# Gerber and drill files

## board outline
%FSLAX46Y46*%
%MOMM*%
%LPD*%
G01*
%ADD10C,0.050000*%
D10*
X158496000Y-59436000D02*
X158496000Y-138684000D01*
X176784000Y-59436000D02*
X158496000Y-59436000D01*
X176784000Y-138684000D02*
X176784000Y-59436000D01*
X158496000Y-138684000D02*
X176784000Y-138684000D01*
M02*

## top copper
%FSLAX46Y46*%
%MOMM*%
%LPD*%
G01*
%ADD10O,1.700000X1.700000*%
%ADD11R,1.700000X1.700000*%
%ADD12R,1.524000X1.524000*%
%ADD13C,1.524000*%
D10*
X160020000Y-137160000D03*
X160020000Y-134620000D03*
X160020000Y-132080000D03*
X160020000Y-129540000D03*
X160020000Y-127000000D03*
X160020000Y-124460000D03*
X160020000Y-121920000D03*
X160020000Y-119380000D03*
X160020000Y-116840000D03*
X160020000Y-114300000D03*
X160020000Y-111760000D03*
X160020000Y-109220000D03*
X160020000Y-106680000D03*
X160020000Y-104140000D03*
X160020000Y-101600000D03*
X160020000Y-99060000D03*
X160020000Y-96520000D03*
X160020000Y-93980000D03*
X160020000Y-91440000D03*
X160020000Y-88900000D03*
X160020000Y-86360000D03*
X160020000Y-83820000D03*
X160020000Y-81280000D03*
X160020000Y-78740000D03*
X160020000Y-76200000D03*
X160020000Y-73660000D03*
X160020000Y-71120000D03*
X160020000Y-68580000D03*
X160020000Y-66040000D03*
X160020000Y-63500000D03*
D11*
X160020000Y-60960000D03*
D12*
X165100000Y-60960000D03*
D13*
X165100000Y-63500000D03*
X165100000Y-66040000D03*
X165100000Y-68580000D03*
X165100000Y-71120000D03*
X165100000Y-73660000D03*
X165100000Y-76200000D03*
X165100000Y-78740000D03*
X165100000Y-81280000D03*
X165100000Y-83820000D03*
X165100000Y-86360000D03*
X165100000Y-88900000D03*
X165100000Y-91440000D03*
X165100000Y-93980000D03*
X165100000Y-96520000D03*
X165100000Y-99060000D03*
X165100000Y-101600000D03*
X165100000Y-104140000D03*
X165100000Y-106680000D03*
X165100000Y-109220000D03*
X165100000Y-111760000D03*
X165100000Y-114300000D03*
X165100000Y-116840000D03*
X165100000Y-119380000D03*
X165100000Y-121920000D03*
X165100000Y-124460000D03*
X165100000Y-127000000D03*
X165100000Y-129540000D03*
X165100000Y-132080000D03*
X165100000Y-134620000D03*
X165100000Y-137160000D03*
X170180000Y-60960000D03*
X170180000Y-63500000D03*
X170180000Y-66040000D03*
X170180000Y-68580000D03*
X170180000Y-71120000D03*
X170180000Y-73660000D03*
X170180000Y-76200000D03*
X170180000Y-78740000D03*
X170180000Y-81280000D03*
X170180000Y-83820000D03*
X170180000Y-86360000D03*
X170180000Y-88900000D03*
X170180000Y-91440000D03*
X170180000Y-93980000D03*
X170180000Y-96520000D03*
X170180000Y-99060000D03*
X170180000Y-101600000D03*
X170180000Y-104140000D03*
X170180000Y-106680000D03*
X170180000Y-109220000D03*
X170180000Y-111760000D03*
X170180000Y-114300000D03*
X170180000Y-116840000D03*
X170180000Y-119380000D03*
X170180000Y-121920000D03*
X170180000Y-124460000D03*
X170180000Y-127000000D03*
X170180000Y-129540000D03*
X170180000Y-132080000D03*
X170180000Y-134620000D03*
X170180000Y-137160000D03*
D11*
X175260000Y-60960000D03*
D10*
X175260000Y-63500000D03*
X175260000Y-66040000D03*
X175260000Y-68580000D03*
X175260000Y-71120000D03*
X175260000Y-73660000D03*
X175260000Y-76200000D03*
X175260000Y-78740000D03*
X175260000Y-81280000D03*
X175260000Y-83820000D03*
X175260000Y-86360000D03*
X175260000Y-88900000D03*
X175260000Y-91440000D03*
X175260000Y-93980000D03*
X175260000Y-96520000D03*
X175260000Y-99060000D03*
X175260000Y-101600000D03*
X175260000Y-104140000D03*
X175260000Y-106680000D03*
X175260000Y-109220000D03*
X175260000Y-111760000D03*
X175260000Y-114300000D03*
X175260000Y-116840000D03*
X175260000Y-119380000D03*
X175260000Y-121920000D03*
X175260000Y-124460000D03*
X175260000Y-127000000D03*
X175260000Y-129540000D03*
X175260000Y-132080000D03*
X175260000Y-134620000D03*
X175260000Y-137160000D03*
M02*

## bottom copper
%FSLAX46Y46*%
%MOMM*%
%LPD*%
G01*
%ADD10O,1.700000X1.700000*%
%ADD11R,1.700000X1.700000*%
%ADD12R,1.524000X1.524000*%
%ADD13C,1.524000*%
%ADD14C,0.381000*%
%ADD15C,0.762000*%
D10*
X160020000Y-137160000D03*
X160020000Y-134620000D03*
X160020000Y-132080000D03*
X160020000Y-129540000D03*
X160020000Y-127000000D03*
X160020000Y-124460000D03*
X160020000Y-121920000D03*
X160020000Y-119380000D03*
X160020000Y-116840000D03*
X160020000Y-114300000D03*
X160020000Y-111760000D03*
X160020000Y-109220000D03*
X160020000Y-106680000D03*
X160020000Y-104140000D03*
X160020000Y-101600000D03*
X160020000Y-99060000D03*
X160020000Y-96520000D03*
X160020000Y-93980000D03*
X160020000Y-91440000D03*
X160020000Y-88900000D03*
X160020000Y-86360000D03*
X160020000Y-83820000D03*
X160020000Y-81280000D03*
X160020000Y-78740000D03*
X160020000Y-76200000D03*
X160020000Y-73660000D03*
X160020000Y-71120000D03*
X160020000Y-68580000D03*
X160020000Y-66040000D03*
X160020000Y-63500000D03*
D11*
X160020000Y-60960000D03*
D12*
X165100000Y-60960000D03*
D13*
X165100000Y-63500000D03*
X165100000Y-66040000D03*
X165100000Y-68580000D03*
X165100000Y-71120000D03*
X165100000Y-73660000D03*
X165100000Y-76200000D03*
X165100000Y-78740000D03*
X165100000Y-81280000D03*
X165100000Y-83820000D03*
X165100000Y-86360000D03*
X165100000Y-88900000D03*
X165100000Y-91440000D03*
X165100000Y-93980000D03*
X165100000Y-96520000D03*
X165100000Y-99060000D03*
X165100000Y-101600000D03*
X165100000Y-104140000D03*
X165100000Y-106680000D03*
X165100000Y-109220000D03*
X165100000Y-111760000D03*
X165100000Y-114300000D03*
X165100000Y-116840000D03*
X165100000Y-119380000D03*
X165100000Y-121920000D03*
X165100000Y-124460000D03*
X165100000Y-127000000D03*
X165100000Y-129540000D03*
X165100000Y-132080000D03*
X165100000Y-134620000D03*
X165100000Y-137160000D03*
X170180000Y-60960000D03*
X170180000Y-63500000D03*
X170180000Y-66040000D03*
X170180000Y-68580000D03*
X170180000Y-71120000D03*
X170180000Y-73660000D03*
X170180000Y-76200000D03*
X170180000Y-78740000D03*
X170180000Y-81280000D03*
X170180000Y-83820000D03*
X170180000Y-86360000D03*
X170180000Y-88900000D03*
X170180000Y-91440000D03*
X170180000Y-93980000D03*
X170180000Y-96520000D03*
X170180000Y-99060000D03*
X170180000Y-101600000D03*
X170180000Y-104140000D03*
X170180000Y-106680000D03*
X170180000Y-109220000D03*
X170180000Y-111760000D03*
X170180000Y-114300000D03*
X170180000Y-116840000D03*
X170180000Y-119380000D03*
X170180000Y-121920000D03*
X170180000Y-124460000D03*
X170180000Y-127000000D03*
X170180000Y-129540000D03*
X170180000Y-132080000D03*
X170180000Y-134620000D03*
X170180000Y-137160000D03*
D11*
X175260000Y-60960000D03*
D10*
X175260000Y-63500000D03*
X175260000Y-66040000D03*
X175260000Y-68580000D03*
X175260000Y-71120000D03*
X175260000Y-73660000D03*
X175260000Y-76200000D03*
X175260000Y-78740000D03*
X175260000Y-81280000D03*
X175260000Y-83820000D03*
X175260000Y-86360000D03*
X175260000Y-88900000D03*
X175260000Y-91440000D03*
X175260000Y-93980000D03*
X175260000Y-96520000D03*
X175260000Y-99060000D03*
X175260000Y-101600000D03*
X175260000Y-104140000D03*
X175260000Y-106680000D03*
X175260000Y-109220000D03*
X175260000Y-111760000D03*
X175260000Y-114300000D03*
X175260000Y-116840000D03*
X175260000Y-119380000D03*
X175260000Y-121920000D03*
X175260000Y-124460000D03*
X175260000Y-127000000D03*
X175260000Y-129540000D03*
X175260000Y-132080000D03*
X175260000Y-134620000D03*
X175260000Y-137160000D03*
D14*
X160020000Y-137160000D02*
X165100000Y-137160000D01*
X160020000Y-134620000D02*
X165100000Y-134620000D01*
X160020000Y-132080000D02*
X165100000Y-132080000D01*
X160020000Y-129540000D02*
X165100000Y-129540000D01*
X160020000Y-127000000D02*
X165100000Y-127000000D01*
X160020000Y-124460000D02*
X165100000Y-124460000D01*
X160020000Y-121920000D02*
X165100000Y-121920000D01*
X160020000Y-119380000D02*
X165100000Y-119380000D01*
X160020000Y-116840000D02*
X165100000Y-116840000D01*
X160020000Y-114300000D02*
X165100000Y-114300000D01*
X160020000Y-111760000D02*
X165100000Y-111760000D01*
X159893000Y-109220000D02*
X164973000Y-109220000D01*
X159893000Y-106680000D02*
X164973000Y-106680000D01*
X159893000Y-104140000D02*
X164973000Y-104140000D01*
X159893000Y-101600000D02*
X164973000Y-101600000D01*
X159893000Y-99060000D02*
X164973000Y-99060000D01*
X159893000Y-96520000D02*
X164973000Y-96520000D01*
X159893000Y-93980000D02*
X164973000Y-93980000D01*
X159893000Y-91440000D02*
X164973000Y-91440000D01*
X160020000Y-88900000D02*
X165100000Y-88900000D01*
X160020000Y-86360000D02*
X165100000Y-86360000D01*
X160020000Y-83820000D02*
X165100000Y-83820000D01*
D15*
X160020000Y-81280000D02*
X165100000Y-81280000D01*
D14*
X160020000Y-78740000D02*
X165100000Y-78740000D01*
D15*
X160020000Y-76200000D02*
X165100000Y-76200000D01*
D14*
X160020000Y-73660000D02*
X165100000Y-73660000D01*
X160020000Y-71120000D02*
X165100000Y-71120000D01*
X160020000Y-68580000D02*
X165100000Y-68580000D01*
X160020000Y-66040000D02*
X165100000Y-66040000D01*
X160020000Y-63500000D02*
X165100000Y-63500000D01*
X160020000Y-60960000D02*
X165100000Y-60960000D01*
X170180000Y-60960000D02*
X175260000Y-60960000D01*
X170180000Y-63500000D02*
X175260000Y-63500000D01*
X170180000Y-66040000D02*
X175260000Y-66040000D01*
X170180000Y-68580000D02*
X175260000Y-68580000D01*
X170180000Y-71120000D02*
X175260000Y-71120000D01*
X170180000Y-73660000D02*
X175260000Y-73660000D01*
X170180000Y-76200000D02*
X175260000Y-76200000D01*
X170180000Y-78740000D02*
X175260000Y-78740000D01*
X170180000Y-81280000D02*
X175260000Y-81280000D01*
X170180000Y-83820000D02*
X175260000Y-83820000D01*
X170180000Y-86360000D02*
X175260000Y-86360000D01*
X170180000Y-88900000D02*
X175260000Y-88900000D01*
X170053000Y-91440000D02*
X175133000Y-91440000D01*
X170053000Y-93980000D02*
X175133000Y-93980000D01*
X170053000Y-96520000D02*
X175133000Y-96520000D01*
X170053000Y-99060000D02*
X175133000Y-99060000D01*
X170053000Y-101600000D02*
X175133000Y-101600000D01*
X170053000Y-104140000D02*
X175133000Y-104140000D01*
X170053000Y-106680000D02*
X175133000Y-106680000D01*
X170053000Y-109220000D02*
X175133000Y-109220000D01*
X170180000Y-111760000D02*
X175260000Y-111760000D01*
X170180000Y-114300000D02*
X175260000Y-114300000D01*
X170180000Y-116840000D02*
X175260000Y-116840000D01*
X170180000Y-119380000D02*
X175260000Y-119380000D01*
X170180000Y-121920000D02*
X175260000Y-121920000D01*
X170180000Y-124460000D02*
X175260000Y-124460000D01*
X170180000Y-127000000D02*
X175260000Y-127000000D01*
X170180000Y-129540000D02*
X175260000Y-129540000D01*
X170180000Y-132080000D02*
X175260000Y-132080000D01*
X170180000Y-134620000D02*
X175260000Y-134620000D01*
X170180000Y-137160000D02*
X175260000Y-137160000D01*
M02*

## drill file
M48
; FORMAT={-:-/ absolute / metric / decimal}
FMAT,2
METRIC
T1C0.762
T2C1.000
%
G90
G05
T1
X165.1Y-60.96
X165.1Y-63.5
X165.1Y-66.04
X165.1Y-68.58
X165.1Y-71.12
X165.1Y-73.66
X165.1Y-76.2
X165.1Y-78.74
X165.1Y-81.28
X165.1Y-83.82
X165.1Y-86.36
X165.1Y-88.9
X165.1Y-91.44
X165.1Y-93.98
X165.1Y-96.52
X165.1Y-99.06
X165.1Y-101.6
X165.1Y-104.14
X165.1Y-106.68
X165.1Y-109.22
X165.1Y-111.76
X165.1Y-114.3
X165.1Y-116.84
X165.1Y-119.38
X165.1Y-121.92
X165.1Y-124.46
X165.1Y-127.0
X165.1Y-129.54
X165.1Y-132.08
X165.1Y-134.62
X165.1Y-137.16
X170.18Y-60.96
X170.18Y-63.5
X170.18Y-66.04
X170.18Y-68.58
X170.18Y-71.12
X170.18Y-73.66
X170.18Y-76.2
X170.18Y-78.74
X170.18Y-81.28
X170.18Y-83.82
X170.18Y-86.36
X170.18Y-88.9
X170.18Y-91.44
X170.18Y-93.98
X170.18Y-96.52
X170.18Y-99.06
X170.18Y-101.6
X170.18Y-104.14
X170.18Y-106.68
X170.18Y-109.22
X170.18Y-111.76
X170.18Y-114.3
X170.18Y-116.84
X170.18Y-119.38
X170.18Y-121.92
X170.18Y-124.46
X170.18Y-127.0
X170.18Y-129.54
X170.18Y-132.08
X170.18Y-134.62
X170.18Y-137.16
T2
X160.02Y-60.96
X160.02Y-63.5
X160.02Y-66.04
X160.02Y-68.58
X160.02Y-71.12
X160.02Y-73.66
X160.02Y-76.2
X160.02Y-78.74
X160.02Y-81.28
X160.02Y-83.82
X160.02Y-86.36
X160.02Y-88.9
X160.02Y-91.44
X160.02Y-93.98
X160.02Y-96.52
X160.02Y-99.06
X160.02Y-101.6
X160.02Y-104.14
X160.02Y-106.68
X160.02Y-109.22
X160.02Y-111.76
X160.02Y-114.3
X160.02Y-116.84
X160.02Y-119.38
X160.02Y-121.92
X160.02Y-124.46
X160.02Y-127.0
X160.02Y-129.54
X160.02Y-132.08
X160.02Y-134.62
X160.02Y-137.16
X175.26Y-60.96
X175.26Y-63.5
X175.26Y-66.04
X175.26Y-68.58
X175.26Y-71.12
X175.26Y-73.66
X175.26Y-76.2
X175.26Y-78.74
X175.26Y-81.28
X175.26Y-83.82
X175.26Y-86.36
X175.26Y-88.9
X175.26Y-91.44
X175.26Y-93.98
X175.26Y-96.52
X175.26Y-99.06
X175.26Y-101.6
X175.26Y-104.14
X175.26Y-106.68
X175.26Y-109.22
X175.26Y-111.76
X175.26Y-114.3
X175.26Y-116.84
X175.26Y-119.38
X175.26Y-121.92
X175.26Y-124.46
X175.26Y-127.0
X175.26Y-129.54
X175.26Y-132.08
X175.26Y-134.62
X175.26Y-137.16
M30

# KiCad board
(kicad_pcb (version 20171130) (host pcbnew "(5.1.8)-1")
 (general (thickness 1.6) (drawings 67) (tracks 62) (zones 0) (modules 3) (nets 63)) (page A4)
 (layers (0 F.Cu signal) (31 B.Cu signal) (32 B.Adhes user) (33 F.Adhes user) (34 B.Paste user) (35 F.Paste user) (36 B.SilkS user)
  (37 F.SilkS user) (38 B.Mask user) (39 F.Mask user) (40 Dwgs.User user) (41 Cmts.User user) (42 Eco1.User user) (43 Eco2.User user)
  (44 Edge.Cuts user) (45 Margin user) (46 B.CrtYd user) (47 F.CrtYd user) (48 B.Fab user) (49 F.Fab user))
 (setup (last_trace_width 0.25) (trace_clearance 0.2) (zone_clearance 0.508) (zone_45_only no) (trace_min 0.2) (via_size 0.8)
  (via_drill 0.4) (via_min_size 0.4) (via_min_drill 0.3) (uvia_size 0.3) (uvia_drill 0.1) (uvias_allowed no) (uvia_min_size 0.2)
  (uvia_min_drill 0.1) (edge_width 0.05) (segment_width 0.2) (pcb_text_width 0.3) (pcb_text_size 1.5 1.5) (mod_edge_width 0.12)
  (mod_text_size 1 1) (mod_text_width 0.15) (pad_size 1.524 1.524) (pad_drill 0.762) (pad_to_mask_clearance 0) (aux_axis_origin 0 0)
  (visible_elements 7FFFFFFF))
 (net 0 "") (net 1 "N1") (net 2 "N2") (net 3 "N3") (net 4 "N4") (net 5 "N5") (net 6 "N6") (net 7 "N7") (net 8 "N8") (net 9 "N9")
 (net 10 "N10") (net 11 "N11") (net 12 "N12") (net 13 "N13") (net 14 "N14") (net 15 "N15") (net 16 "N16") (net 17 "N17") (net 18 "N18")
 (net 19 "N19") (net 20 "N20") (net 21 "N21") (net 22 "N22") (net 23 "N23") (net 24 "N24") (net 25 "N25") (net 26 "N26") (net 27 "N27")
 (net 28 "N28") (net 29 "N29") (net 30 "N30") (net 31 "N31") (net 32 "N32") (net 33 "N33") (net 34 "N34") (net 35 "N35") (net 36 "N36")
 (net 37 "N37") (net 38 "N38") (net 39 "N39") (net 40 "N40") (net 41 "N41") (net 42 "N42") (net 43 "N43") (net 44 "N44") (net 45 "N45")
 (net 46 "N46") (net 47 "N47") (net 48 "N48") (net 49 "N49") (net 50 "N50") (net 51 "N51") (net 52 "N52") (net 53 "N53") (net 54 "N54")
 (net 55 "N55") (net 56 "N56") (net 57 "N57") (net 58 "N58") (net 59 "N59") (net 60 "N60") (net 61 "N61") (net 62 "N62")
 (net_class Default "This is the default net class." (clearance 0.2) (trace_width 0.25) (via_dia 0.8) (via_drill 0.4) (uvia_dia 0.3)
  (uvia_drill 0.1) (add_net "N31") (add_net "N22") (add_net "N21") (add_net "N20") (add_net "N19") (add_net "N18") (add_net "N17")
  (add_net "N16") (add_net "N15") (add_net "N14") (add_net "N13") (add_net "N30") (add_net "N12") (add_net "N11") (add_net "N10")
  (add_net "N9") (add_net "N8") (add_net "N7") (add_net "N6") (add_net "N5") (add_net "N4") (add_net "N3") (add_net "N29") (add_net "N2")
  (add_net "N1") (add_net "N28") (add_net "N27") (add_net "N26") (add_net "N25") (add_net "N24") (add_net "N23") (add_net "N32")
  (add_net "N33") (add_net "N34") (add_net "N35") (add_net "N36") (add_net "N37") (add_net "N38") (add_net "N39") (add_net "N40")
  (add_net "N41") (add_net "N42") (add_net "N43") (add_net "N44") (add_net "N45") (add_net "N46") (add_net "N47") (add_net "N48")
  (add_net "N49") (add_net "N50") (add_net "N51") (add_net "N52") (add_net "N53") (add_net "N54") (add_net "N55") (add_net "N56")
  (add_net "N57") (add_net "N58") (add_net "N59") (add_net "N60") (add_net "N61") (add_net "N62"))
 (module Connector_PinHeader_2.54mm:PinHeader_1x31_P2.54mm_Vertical (layer B.Cu) (at 160.02 60.96 180)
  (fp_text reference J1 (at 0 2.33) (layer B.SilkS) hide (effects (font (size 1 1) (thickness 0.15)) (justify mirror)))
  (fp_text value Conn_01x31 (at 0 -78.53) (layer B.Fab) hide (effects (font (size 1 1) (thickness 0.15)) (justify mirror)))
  (pad 31 thru_hole oval (at 0 -76.2 180) (size 1.7 1.7) (drill 1) (layers *.Cu *.Mask) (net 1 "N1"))
  (pad 30 thru_hole oval (at 0 -73.66 180) (size 1.7 1.7) (drill 1) (layers *.Cu *.Mask) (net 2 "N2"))
  (pad 29 thru_hole oval (at 0 -71.12 180) (size 1.7 1.7) (drill 1) (layers *.Cu *.Mask) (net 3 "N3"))
  (pad 28 thru_hole oval (at 0 -68.58 180) (size 1.7 1.7) (drill 1) (layers *.Cu *.Mask) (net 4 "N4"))
  (pad 27 thru_hole oval (at 0 -66.04 180) (size 1.7 1.7) (drill 1) (layers *.Cu *.Mask) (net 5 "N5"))
  (pad 26 thru_hole oval (at 0 -63.5 180) (size 1.7 1.7) (drill 1) (layers *.Cu *.Mask) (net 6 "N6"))
  (pad 25 thru_hole oval (at 0 -60.96 180) (size 1.7 1.7) (drill 1) (layers *.Cu *.Mask) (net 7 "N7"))
  (pad 24 thru_hole oval (at 0 -58.42 180) (size 1.7 1.7) (drill 1) (layers *.Cu *.Mask) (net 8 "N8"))
  (pad 23 thru_hole oval (at 0 -55.88 180) (size 1.7 1.7) (drill 1) (layers *.Cu *.Mask) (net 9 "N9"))
  (pad 22 thru_hole oval (at 0 -53.34 180) (size 1.7 1.7) (drill 1) (layers *.Cu *.Mask) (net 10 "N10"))
  (pad 21 thru_hole oval (at 0 -50.8 180) (size 1.7 1.7) (drill 1) (layers *.Cu *.Mask) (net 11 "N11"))
  (pad 20 thru_hole oval (at 0 -48.26 180) (size 1.7 1.7) (drill 1) (layers *.Cu *.Mask) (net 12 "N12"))
  (pad 19 thru_hole oval (at 0 -45.72 180) (size 1.7 1.7) (drill 1) (layers *.Cu *.Mask) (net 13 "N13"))
  (pad 18 thru_hole oval (at 0 -43.18 180) (size 1.7 1.7) (drill 1) (layers *.Cu *.Mask) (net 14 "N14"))
  (pad 17 thru_hole oval (at 0 -40.64 180) (size 1.7 1.7) (drill 1) (layers *.Cu *.Mask) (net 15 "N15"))
  (pad 16 thru_hole oval (at 0 -38.1 180) (size 1.7 1.7) (drill 1) (layers *.Cu *.Mask) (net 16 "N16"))
  (pad 15 thru_hole oval (at 0 -35.56 180) (size 1.7 1.7) (drill 1) (layers *.Cu *.Mask) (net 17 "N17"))
  (pad 14 thru_hole oval (at 0 -33.02 180) (size 1.7 1.7) (drill 1) (layers *.Cu *.Mask) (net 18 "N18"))
  (pad 13 thru_hole oval (at 0 -30.48 180) (size 1.7 1.7) (drill 1) (layers *.Cu *.Mask) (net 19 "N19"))
  (pad 12 thru_hole oval (at 0 -27.94 180) (size 1.7 1.7) (drill 1) (layers *.Cu *.Mask) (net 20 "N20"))
  (pad 11 thru_hole oval (at 0 -25.4 180) (size 1.7 1.7) (drill 1) (layers *.Cu *.Mask) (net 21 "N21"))
  (pad 10 thru_hole oval (at 0 -22.86 180) (size 1.7 1.7) (drill 1) (layers *.Cu *.Mask) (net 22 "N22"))
  (pad 9 thru_hole oval (at 0 -20.32 180) (size 1.7 1.7) (drill 1) (layers *.Cu *.Mask) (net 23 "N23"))
  (pad 8 thru_hole oval (at 0 -17.78 180) (size 1.7 1.7) (drill 1) (layers *.Cu *.Mask) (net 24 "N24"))
  (pad 7 thru_hole oval (at 0 -15.24 180) (size 1.7 1.7) (drill 1) (layers *.Cu *.Mask) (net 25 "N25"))
  (pad 6 thru_hole oval (at 0 -12.7 180) (size 1.7 1.7) (drill 1) (layers *.Cu *.Mask) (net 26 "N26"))
  (pad 5 thru_hole oval (at 0 -10.16 180) (size 1.7 1.7) (drill 1) (layers *.Cu *.Mask) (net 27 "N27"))
  (pad 4 thru_hole oval (at 0 -7.62 180) (size 1.7 1.7) (drill 1) (layers *.Cu *.Mask) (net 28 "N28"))
  (pad 3 thru_hole oval (at 0 -5.08 180) (size 1.7 1.7) (drill 1) (layers *.Cu *.Mask) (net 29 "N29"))
  (pad 2 thru_hole oval (at 0 -2.54 180) (size 1.7 1.7) (drill 1) (layers *.Cu *.Mask) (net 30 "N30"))
  (pad 1 thru_hole rect (at 0 0 180) (size 1.7 1.7) (drill 1) (layers *.Cu *.Mask) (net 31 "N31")))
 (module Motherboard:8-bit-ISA (layer F.Cu) (at 165.1 60.96)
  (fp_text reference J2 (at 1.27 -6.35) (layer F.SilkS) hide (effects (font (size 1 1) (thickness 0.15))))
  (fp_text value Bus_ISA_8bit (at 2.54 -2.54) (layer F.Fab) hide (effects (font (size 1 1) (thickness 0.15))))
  (pad 1 thru_hole rect (at 0 0) (size 1.524 1.524) (drill 0.762) (layers *.Cu *.Mask) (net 31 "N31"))
  (pad 2 thru_hole circle (at 0 2.54) (size 1.524 1.524) (drill 0.762) (layers *.Cu *.Mask) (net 30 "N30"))
  (pad 3 thru_hole circle (at 0 5.08) (size 1.524 1.524) (drill 0.762) (layers *.Cu *.Mask) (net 29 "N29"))
  (pad 4 thru_hole circle (at 0 7.62) (size 1.524 1.524) (drill 0.762) (layers *.Cu *.Mask) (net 28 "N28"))
  (pad 5 thru_hole circle (at 0 10.16) (size 1.524 1.524) (drill 0.762) (layers *.Cu *.Mask) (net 27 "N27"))
  (pad 6 thru_hole circle (at 0 12.7) (size 1.524 1.524) (drill 0.762) (layers *.Cu *.Mask) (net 26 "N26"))
  (pad 7 thru_hole circle (at 0 15.24) (size 1.524 1.524) (drill 0.762) (layers *.Cu *.Mask) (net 25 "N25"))
  (pad 8 thru_hole circle (at 0 17.78) (size 1.524 1.524) (drill 0.762) (layers *.Cu *.Mask) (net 24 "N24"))
  (pad 9 thru_hole circle (at 0 20.32) (size 1.524 1.524) (drill 0.762) (layers *.Cu *.Mask) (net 23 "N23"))
  (pad 10 thru_hole circle (at 0 22.86) (size 1.524 1.524) (drill 0.762) (layers *.Cu *.Mask) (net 22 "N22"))
  (pad 11 thru_hole circle (at 0 25.4) (size 1.524 1.524) (drill 0.762) (layers *.Cu *.Mask) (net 21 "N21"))
  (pad 12 thru_hole circle (at 0 27.94) (size 1.524 1.524) (drill 0.762) (layers *.Cu *.Mask) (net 20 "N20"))
  (pad 13 thru_hole circle (at 0 30.48) (size 1.524 1.524) (drill 0.762) (layers *.Cu *.Mask) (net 19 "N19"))
  (pad 14 thru_hole circle (at 0 33.02) (size 1.524 1.524) (drill 0.762) (layers *.Cu *.Mask) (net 18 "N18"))
  (pad 15 thru_hole circle (at 0 35.56) (size 1.524 1.524) (drill 0.762) (layers *.Cu *.Mask) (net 17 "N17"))
  (pad 16 thru_hole circle (at 0 38.1) (size 1.524 1.524) (drill 0.762) (layers *.Cu *.Mask) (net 16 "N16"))
  (pad 17 thru_hole circle (at 0 40.64) (size 1.524 1.524) (drill 0.762) (layers *.Cu *.Mask) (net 15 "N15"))
  (pad 18 thru_hole circle (at 0 43.18) (size 1.524 1.524) (drill 0.762) (layers *.Cu *.Mask) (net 14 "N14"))
  (pad 19 thru_hole circle (at 0 45.72) (size 1.524 1.524) (drill 0.762) (layers *.Cu *.Mask) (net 13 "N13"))
  (pad 20 thru_hole circle (at 0 48.26) (size 1.524 1.524) (drill 0.762) (layers *.Cu *.Mask) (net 12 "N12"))
  (pad 21 thru_hole circle (at 0 50.8) (size 1.524 1.524) (drill 0.762) (layers *.Cu *.Mask) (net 11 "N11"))
  (pad 22 thru_hole circle (at 0 53.34) (size 1.524 1.524) (drill 0.762) (layers *.Cu *.Mask) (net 10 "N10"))
  (pad 23 thru_hole circle (at 0 55.88) (size 1.524 1.524) (drill 0.762) (layers *.Cu *.Mask) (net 9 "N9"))
  (pad 24 thru_hole circle (at 0 58.42) (size 1.524 1.524) (drill 0.762) (layers *.Cu *.Mask) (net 8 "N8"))
  (pad 25 thru_hole circle (at 0 60.96) (size 1.524 1.524) (drill 0.762) (layers *.Cu *.Mask) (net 7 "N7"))
  (pad 26 thru_hole circle (at 0 63.5) (size 1.524 1.524) (drill 0.762) (layers *.Cu *.Mask) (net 6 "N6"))
  (pad 27 thru_hole circle (at 0 66.04) (size 1.524 1.524) (drill 0.762) (layers *.Cu *.Mask) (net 5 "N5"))
  (pad 28 thru_hole circle (at 0 68.58) (size 1.524 1.524) (drill 0.762) (layers *.Cu *.Mask) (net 4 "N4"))
  (pad 29 thru_hole circle (at 0 71.12) (size 1.524 1.524) (drill 0.762) (layers *.Cu *.Mask) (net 3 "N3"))
  (pad 30 thru_hole circle (at 0 73.66) (size 1.524 1.524) (drill 0.762) (layers *.Cu *.Mask) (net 2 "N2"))
  (pad 31 thru_hole circle (at 0 76.2) (size 1.524 1.524) (drill 0.762) (layers *.Cu *.Mask) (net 1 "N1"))
  (pad 32 thru_hole circle (at 5.08 0) (size 1.524 1.524) (drill 0.762) (layers *.Cu *.Mask) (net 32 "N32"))
  (pad 33 thru_hole circle (at 5.08 2.54) (size 1.524 1.524) (drill 0.762) (layers *.Cu *.Mask) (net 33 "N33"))
  (pad 34 thru_hole circle (at 5.08 5.08) (size 1.524 1.524) (drill 0.762) (layers *.Cu *.Mask) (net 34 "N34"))
  (pad 35 thru_hole circle (at 5.08 7.62) (size 1.524 1.524) (drill 0.762) (layers *.Cu *.Mask) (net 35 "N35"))
  (pad 36 thru_hole circle (at 5.08 10.16) (size 1.524 1.524) (drill 0.762) (layers *.Cu *.Mask) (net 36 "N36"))
  (pad 37 thru_hole circle (at 5.08 12.7) (size 1.524 1.524) (drill 0.762) (layers *.Cu *.Mask) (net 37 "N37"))
  (pad 38 thru_hole circle (at 5.08 15.24) (size 1.524 1.524) (drill 0.762) (layers *.Cu *.Mask) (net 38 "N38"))
  (pad 39 thru_hole circle (at 5.08 17.78) (size 1.524 1.524) (drill 0.762) (layers *.Cu *.Mask) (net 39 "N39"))
  (pad 40 thru_hole circle (at 5.08 20.32) (size 1.524 1.524) (drill 0.762) (layers *.Cu *.Mask) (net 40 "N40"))
  (pad 41 thru_hole circle (at 5.08 22.86) (size 1.524 1.524) (drill 0.762) (layers *.Cu *.Mask) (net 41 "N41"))
  (pad 42 thru_hole circle (at 5.08 25.4) (size 1.524 1.524) (drill 0.762) (layers *.Cu *.Mask) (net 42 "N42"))
  (pad 43 thru_hole circle (at 5.08 27.94) (size 1.524 1.524) (drill 0.762) (layers *.Cu *.Mask) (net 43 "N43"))
  (pad 44 thru_hole circle (at 5.08 30.48) (size 1.524 1.524) (drill 0.762) (layers *.Cu *.Mask) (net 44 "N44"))
  (pad 45 thru_hole circle (at 5.08 33.02) (size 1.524 1.524) (drill 0.762) (layers *.Cu *.Mask) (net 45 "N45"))
  (pad 46 thru_hole circle (at 5.08 35.56) (size 1.524 1.524) (drill 0.762) (layers *.Cu *.Mask) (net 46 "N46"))
  (pad 47 thru_hole circle (at 5.08 38.1) (size 1.524 1.524) (drill 0.762) (layers *.Cu *.Mask) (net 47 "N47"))
  (pad 48 thru_hole circle (at 5.08 40.64) (size 1.524 1.524) (drill 0.762) (layers *.Cu *.Mask) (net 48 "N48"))
  (pad 49 thru_hole circle (at 5.08 43.18) (size 1.524 1.524) (drill 0.762) (layers *.Cu *.Mask) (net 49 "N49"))
  (pad 50 thru_hole circle (at 5.08 45.72) (size 1.524 1.524) (drill 0.762) (layers *.Cu *.Mask) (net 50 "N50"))
  (pad 51 thru_hole circle (at 5.08 48.26) (size 1.524 1.524) (drill 0.762) (layers *.Cu *.Mask) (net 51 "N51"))
  (pad 52 thru_hole circle (at 5.08 50.8) (size 1.524 1.524) (drill 0.762) (layers *.Cu *.Mask) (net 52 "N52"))
  (pad 53 thru_hole circle (at 5.08 53.34) (size 1.524 1.524) (drill 0.762) (layers *.Cu *.Mask) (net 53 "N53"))
  (pad 54 thru_hole circle (at 5.08 55.88) (size 1.524 1.524) (drill 0.762) (layers *.Cu *.Mask) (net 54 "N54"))
  (pad 55 thru_hole circle (at 5.08 58.42) (size 1.524 1.524) (drill 0.762) (layers *.Cu *.Mask) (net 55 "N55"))
  (pad 56 thru_hole circle (at 5.08 60.96) (size 1.524 1.524) (drill 0.762) (layers *.Cu *.Mask) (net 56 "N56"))
  (pad 57 thru_hole circle (at 5.08 63.5) (size 1.524 1.524) (drill 0.762) (layers *.Cu *.Mask) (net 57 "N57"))
  (pad 58 thru_hole circle (at 5.08 66.04) (size 1.524 1.524) (drill 0.762) (layers *.Cu *.Mask) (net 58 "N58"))
  (pad 59 thru_hole circle (at 5.08 68.58) (size 1.524 1.524) (drill 0.762) (layers *.Cu *.Mask) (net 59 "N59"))
  (pad 60 thru_hole circle (at 5.08 71.12) (size 1.524 1.524) (drill 0.762) (layers *.Cu *.Mask) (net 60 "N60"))
  (pad 61 thru_hole circle (at 5.08 73.66) (size 1.524 1.524) (drill 0.762) (layers *.Cu *.Mask) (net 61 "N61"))
  (pad 62 thru_hole circle (at 5.08 76.2) (size 1.524 1.524) (drill 0.762) (layers *.Cu *.Mask) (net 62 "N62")))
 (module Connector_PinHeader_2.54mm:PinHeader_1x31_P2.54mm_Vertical (layer B.Cu) (at 175.26 60.96 180)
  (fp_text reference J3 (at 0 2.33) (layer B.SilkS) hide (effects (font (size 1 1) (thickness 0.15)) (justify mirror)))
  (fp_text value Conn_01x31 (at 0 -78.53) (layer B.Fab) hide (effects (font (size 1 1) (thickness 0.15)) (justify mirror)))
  (pad 1 thru_hole rect (at 0 0 180) (size 1.7 1.7) (drill 1) (layers *.Cu *.Mask) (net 32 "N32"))
  (pad 2 thru_hole oval (at 0 -2.54 180) (size 1.7 1.7) (drill 1) (layers *.Cu *.Mask) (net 33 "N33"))
  (pad 3 thru_hole oval (at 0 -5.08 180) (size 1.7 1.7) (drill 1) (layers *.Cu *.Mask) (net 34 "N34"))
  (pad 4 thru_hole oval (at 0 -7.62 180) (size 1.7 1.7) (drill 1) (layers *.Cu *.Mask) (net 35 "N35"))
  (pad 5 thru_hole oval (at 0 -10.16 180) (size 1.7 1.7) (drill 1) (layers *.Cu *.Mask) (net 36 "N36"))
  (pad 6 thru_hole oval (at 0 -12.7 180) (size 1.7 1.7) (drill 1) (layers *.Cu *.Mask) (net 37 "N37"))
  (pad 7 thru_hole oval (at 0 -15.24 180) (size 1.7 1.7) (drill 1) (layers *.Cu *.Mask) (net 38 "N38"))
  (pad 8 thru_hole oval (at 0 -17.78 180) (size 1.7 1.7) (drill 1) (layers *.Cu *.Mask) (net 39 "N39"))
  (pad 9 thru_hole oval (at 0 -20.32 180) (size 1.7 1.7) (drill 1) (layers *.Cu *.Mask) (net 40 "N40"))
  (pad 10 thru_hole oval (at 0 -22.86 180) (size 1.7 1.7) (drill 1) (layers *.Cu *.Mask) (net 41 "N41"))
  (pad 11 thru_hole oval (at 0 -25.4 180) (size 1.7 1.7) (drill 1) (layers *.Cu *.Mask) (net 42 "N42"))
  (pad 12 thru_hole oval (at 0 -27.94 180) (size 1.7 1.7) (drill 1) (layers *.Cu *.Mask) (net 43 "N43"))
  (pad 13 thru_hole oval (at 0 -30.48 180) (size 1.7 1.7) (drill 1) (layers *.Cu *.Mask) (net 44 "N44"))
  (pad 14 thru_hole oval (at 0 -33.02 180) (size 1.7 1.7) (drill 1) (layers *.Cu *.Mask) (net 45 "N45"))
  (pad 15 thru_hole oval (at 0 -35.56 180) (size 1.7 1.7) (drill 1) (layers *.Cu *.Mask) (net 46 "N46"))
  (pad 16 thru_hole oval (at 0 -38.1 180) (size 1.7 1.7) (drill 1) (layers *.Cu *.Mask) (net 47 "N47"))
  (pad 17 thru_hole oval (at 0 -40.64 180) (size 1.7 1.7) (drill 1) (layers *.Cu *.Mask) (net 48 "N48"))
  (pad 18 thru_hole oval (at 0 -43.18 180) (size 1.7 1.7) (drill 1) (layers *.Cu *.Mask) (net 49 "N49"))
  (pad 19 thru_hole oval (at 0 -45.72 180) (size 1.7 1.7) (drill 1) (layers *.Cu *.Mask) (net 50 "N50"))
  (pad 20 thru_hole oval (at 0 -48.26 180) (size 1.7 1.7) (drill 1) (layers *.Cu *.Mask) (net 51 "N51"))
  (pad 21 thru_hole oval (at 0 -50.8 180) (size 1.7 1.7) (drill 1) (layers *.Cu *.Mask) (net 52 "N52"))
  (pad 22 thru_hole oval (at 0 -53.34 180) (size 1.7 1.7) (drill 1) (layers *.Cu *.Mask) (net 53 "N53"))
  (pad 23 thru_hole oval (at 0 -55.88 180) (size 1.7 1.7) (drill 1) (layers *.Cu *.Mask) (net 54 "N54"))
  (pad 24 thru_hole oval (at 0 -58.42 180) (size 1.7 1.7) (drill 1) (layers *.Cu *.Mask) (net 55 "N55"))
  (pad 25 thru_hole oval (at 0 -60.96 180) (size 1.7 1.7) (drill 1) (layers *.Cu *.Mask) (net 56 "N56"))
  (pad 26 thru_hole oval (at 0 -63.5 180) (size 1.7 1.7) (drill 1) (layers *.Cu *.Mask) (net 57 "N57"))
  (pad 27 thru_hole oval (at 0 -66.04 180) (size 1.7 1.7) (drill 1) (layers *.Cu *.Mask) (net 58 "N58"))
  (pad 28 thru_hole oval (at 0 -68.58 180) (size 1.7 1.7) (drill 1) (layers *.Cu *.Mask) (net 59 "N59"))
  (pad 29 thru_hole oval (at 0 -71.12 180) (size 1.7 1.7) (drill 1) (layers *.Cu *.Mask) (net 60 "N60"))
  (pad 30 thru_hole oval (at 0 -73.66 180) (size 1.7 1.7) (drill 1) (layers *.Cu *.Mask) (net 61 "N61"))
  (pad 31 thru_hole oval (at 0 -76.2 180) (size 1.7 1.7) (drill 1) (layers *.Cu *.Mask) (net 62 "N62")))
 (gr_line (start 158.496 59.436) (end 158.496 138.684) (layer Edge.Cuts) (width 0.05))
 (gr_line (start 176.784 59.436) (end 158.496 59.436) (layer Edge.Cuts) (width 0.05))
 (gr_line (start 176.784 138.684) (end 176.784 59.436) (layer Edge.Cuts) (width 0.05))
 (gr_line (start 158.496 138.684) (end 176.784 138.684) (layer Edge.Cuts) (width 0.05))
 (segment (start 160.02 137.16) (end 165.1 137.16) (width 0.381) (layer B.Cu) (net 1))
 (segment (start 160.02 134.62) (end 165.1 134.62) (width 0.381) (layer B.Cu) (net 2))
 (segment (start 160.02 132.08) (end 165.1 132.08) (width 0.381) (layer B.Cu) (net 3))
 (segment (start 160.02 129.54) (end 165.1 129.54) (width 0.381) (layer B.Cu) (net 4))
 (segment (start 160.02 127) (end 165.1 127) (width 0.381) (layer B.Cu) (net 5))
 (segment (start 160.02 124.46) (end 165.1 124.46) (width 0.381) (layer B.Cu) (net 6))
 (segment (start 160.02 121.92) (end 165.1 121.92) (width 0.381) (layer B.Cu) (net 7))
 (segment (start 160.02 119.38) (end 165.1 119.38) (width 0.381) (layer B.Cu) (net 8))
 (segment (start 160.02 116.84) (end 165.1 116.84) (width 0.381) (layer B.Cu) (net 9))
 (segment (start 160.02 114.3) (end 165.1 114.3) (width 0.381) (layer B.Cu) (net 10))
 (segment (start 160.02 111.76) (end 165.1 111.76) (width 0.381) (layer B.Cu) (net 11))
 (segment (start 159.893 109.22) (end 164.973 109.22) (width 0.381) (layer B.Cu) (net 12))
 (segment (start 159.893 106.68) (end 164.973 106.68) (width 0.381) (layer B.Cu) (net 13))
 (segment (start 159.893 104.14) (end 164.973 104.14) (width 0.381) (layer B.Cu) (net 14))
 (segment (start 159.893 101.6) (end 164.973 101.6) (width 0.381) (layer B.Cu) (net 15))
 (segment (start 159.893 99.06) (end 164.973 99.06) (width 0.381) (layer B.Cu) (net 16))
 (segment (start 159.893 96.52) (end 164.973 96.52) (width 0.381) (layer B.Cu) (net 17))
 (segment (start 159.893 93.98) (end 164.973 93.98) (width 0.381) (layer B.Cu) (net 18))
 (segment (start 159.893 91.44) (end 164.973 91.44) (width 0.381) (layer B.Cu) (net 19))
 (segment (start 160.02 88.9) (end 165.1 88.9) (width 0.381) (layer B.Cu) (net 20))
 (segment (start 160.02 86.36) (end 165.1 86.36) (width 0.381) (layer B.Cu) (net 21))
 (segment (start 160.02 83.82) (end 165.1 83.82) (width 0.381) (layer B.Cu) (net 22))
 (segment (start 160.02 81.28) (end 165.1 81.28) (width 0.762) (layer B.Cu) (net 23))
 (segment (start 160.02 78.74) (end 165.1 78.74) (width 0.381) (layer B.Cu) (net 24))
 (segment (start 160.02 76.2) (end 165.1 76.2) (width 0.762) (layer B.Cu) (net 25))
 (segment (start 160.02 73.66) (end 165.1 73.66) (width 0.381) (layer B.Cu) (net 26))
 (segment (start 160.02 71.12) (end 165.1 71.12) (width 0.381) (layer B.Cu) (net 27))
 (segment (start 160.02 68.58) (end 165.1 68.58) (width 0.381) (layer B.Cu) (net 28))
 (segment (start 160.02 66.04) (end 165.1 66.04) (width 0.381) (layer B.Cu) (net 29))
 (segment (start 160.02 63.5) (end 165.1 63.5) (width 0.381) (layer B.Cu) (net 30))
 (segment (start 160.02 60.96) (end 165.1 60.96) (width 0.381) (layer B.Cu) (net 31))
 (segment (start 170.18 60.96) (end 175.26 60.96) (width 0.381) (layer B.Cu) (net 32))
 (segment (start 170.18 63.5) (end 175.26 63.5) (width 0.381) (layer B.Cu) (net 33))
 (segment (start 170.18 66.04) (end 175.26 66.04) (width 0.381) (layer B.Cu) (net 34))
 (segment (start 170.18 68.58) (end 175.26 68.58) (width 0.381) (layer B.Cu) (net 35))
 (segment (start 170.18 71.12) (end 175.26 71.12) (width 0.381) (layer B.Cu) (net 36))
 (segment (start 170.18 73.66) (end 175.26 73.66) (width 0.381) (layer B.Cu) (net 37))
 (segment (start 170.18 76.2) (end 175.26 76.2) (width 0.381) (layer B.Cu) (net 38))
 (segment (start 170.18 78.74) (end 175.26 78.74) (width 0.381) (layer B.Cu) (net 39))
 (segment (start 170.18 81.28) (end 175.26 81.28) (width 0.381) (layer B.Cu) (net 40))
 (segment (start 170.18 83.82) (end 175.26 83.82) (width 0.381) (layer B.Cu) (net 41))
 (segment (start 170.18 86.36) (end 175.26 86.36) (width 0.381) (layer B.Cu) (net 42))
 (segment (start 170.18 88.9) (end 175.26 88.9) (width 0.381) (layer B.Cu) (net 43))
 (segment (start 170.053 91.44) (end 175.133 91.44) (width 0.381) (layer B.Cu) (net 44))
 (segment (start 170.053 93.98) (end 175.133 93.98) (width 0.381) (layer B.Cu) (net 45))
 (segment (start 170.053 96.52) (end 175.133 96.52) (width 0.381) (layer B.Cu) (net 46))
 (segment (start 170.053 99.06) (end 175.133 99.06) (width 0.381) (layer B.Cu) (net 47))
 (segment (start 170.053 101.6) (end 175.133 101.6) (width 0.381) (layer B.Cu) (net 48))
 (segment (start 170.053 104.14) (end 175.133 104.14) (width 0.381) (layer B.Cu) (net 49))
 (segment (start 170.053 106.68) (end 175.133 106.68) (width 0.381) (layer B.Cu) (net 50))
 (segment (start 170.053 109.22) (end 175.133 109.22) (width 0.381) (layer B.Cu) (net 51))
 (segment (start 170.18 111.76) (end 175.26 111.76) (width 0.381) (layer B.Cu) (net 52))
 (segment (start 170.18 114.3) (end 175.26 114.3) (width 0.381) (layer B.Cu) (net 53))
 (segment (start 170.18 116.84) (end 175.26 116.84) (width 0.381) (layer B.Cu) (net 54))
 (segment (start 170.18 119.38) (end 175.26 119.38) (width 0.381) (layer B.Cu) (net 55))
 (segment (start 170.18 121.92) (end 175.26 121.92) (width 0.381) (layer B.Cu) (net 56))
 (segment (start 170.18 124.46) (end 175.26 124.46) (width 0.381) (layer B.Cu) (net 57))
 (segment (start 170.18 127) (end 175.26 127) (width 0.381) (layer B.Cu) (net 58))
 (segment (start 170.18 129.54) (end 175.26 129.54) (width 0.381) (layer B.Cu) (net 59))
 (segment (start 170.18 132.08) (end 175.26 132.08) (width 0.381) (layer B.Cu) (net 60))
 (segment (start 170.18 134.62) (end 175.26 134.62) (width 0.381) (layer B.Cu) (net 61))
 (segment (start 170.18 137.16) (end 175.26 137.16) (width 0.381) (layer B.Cu) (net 62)))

